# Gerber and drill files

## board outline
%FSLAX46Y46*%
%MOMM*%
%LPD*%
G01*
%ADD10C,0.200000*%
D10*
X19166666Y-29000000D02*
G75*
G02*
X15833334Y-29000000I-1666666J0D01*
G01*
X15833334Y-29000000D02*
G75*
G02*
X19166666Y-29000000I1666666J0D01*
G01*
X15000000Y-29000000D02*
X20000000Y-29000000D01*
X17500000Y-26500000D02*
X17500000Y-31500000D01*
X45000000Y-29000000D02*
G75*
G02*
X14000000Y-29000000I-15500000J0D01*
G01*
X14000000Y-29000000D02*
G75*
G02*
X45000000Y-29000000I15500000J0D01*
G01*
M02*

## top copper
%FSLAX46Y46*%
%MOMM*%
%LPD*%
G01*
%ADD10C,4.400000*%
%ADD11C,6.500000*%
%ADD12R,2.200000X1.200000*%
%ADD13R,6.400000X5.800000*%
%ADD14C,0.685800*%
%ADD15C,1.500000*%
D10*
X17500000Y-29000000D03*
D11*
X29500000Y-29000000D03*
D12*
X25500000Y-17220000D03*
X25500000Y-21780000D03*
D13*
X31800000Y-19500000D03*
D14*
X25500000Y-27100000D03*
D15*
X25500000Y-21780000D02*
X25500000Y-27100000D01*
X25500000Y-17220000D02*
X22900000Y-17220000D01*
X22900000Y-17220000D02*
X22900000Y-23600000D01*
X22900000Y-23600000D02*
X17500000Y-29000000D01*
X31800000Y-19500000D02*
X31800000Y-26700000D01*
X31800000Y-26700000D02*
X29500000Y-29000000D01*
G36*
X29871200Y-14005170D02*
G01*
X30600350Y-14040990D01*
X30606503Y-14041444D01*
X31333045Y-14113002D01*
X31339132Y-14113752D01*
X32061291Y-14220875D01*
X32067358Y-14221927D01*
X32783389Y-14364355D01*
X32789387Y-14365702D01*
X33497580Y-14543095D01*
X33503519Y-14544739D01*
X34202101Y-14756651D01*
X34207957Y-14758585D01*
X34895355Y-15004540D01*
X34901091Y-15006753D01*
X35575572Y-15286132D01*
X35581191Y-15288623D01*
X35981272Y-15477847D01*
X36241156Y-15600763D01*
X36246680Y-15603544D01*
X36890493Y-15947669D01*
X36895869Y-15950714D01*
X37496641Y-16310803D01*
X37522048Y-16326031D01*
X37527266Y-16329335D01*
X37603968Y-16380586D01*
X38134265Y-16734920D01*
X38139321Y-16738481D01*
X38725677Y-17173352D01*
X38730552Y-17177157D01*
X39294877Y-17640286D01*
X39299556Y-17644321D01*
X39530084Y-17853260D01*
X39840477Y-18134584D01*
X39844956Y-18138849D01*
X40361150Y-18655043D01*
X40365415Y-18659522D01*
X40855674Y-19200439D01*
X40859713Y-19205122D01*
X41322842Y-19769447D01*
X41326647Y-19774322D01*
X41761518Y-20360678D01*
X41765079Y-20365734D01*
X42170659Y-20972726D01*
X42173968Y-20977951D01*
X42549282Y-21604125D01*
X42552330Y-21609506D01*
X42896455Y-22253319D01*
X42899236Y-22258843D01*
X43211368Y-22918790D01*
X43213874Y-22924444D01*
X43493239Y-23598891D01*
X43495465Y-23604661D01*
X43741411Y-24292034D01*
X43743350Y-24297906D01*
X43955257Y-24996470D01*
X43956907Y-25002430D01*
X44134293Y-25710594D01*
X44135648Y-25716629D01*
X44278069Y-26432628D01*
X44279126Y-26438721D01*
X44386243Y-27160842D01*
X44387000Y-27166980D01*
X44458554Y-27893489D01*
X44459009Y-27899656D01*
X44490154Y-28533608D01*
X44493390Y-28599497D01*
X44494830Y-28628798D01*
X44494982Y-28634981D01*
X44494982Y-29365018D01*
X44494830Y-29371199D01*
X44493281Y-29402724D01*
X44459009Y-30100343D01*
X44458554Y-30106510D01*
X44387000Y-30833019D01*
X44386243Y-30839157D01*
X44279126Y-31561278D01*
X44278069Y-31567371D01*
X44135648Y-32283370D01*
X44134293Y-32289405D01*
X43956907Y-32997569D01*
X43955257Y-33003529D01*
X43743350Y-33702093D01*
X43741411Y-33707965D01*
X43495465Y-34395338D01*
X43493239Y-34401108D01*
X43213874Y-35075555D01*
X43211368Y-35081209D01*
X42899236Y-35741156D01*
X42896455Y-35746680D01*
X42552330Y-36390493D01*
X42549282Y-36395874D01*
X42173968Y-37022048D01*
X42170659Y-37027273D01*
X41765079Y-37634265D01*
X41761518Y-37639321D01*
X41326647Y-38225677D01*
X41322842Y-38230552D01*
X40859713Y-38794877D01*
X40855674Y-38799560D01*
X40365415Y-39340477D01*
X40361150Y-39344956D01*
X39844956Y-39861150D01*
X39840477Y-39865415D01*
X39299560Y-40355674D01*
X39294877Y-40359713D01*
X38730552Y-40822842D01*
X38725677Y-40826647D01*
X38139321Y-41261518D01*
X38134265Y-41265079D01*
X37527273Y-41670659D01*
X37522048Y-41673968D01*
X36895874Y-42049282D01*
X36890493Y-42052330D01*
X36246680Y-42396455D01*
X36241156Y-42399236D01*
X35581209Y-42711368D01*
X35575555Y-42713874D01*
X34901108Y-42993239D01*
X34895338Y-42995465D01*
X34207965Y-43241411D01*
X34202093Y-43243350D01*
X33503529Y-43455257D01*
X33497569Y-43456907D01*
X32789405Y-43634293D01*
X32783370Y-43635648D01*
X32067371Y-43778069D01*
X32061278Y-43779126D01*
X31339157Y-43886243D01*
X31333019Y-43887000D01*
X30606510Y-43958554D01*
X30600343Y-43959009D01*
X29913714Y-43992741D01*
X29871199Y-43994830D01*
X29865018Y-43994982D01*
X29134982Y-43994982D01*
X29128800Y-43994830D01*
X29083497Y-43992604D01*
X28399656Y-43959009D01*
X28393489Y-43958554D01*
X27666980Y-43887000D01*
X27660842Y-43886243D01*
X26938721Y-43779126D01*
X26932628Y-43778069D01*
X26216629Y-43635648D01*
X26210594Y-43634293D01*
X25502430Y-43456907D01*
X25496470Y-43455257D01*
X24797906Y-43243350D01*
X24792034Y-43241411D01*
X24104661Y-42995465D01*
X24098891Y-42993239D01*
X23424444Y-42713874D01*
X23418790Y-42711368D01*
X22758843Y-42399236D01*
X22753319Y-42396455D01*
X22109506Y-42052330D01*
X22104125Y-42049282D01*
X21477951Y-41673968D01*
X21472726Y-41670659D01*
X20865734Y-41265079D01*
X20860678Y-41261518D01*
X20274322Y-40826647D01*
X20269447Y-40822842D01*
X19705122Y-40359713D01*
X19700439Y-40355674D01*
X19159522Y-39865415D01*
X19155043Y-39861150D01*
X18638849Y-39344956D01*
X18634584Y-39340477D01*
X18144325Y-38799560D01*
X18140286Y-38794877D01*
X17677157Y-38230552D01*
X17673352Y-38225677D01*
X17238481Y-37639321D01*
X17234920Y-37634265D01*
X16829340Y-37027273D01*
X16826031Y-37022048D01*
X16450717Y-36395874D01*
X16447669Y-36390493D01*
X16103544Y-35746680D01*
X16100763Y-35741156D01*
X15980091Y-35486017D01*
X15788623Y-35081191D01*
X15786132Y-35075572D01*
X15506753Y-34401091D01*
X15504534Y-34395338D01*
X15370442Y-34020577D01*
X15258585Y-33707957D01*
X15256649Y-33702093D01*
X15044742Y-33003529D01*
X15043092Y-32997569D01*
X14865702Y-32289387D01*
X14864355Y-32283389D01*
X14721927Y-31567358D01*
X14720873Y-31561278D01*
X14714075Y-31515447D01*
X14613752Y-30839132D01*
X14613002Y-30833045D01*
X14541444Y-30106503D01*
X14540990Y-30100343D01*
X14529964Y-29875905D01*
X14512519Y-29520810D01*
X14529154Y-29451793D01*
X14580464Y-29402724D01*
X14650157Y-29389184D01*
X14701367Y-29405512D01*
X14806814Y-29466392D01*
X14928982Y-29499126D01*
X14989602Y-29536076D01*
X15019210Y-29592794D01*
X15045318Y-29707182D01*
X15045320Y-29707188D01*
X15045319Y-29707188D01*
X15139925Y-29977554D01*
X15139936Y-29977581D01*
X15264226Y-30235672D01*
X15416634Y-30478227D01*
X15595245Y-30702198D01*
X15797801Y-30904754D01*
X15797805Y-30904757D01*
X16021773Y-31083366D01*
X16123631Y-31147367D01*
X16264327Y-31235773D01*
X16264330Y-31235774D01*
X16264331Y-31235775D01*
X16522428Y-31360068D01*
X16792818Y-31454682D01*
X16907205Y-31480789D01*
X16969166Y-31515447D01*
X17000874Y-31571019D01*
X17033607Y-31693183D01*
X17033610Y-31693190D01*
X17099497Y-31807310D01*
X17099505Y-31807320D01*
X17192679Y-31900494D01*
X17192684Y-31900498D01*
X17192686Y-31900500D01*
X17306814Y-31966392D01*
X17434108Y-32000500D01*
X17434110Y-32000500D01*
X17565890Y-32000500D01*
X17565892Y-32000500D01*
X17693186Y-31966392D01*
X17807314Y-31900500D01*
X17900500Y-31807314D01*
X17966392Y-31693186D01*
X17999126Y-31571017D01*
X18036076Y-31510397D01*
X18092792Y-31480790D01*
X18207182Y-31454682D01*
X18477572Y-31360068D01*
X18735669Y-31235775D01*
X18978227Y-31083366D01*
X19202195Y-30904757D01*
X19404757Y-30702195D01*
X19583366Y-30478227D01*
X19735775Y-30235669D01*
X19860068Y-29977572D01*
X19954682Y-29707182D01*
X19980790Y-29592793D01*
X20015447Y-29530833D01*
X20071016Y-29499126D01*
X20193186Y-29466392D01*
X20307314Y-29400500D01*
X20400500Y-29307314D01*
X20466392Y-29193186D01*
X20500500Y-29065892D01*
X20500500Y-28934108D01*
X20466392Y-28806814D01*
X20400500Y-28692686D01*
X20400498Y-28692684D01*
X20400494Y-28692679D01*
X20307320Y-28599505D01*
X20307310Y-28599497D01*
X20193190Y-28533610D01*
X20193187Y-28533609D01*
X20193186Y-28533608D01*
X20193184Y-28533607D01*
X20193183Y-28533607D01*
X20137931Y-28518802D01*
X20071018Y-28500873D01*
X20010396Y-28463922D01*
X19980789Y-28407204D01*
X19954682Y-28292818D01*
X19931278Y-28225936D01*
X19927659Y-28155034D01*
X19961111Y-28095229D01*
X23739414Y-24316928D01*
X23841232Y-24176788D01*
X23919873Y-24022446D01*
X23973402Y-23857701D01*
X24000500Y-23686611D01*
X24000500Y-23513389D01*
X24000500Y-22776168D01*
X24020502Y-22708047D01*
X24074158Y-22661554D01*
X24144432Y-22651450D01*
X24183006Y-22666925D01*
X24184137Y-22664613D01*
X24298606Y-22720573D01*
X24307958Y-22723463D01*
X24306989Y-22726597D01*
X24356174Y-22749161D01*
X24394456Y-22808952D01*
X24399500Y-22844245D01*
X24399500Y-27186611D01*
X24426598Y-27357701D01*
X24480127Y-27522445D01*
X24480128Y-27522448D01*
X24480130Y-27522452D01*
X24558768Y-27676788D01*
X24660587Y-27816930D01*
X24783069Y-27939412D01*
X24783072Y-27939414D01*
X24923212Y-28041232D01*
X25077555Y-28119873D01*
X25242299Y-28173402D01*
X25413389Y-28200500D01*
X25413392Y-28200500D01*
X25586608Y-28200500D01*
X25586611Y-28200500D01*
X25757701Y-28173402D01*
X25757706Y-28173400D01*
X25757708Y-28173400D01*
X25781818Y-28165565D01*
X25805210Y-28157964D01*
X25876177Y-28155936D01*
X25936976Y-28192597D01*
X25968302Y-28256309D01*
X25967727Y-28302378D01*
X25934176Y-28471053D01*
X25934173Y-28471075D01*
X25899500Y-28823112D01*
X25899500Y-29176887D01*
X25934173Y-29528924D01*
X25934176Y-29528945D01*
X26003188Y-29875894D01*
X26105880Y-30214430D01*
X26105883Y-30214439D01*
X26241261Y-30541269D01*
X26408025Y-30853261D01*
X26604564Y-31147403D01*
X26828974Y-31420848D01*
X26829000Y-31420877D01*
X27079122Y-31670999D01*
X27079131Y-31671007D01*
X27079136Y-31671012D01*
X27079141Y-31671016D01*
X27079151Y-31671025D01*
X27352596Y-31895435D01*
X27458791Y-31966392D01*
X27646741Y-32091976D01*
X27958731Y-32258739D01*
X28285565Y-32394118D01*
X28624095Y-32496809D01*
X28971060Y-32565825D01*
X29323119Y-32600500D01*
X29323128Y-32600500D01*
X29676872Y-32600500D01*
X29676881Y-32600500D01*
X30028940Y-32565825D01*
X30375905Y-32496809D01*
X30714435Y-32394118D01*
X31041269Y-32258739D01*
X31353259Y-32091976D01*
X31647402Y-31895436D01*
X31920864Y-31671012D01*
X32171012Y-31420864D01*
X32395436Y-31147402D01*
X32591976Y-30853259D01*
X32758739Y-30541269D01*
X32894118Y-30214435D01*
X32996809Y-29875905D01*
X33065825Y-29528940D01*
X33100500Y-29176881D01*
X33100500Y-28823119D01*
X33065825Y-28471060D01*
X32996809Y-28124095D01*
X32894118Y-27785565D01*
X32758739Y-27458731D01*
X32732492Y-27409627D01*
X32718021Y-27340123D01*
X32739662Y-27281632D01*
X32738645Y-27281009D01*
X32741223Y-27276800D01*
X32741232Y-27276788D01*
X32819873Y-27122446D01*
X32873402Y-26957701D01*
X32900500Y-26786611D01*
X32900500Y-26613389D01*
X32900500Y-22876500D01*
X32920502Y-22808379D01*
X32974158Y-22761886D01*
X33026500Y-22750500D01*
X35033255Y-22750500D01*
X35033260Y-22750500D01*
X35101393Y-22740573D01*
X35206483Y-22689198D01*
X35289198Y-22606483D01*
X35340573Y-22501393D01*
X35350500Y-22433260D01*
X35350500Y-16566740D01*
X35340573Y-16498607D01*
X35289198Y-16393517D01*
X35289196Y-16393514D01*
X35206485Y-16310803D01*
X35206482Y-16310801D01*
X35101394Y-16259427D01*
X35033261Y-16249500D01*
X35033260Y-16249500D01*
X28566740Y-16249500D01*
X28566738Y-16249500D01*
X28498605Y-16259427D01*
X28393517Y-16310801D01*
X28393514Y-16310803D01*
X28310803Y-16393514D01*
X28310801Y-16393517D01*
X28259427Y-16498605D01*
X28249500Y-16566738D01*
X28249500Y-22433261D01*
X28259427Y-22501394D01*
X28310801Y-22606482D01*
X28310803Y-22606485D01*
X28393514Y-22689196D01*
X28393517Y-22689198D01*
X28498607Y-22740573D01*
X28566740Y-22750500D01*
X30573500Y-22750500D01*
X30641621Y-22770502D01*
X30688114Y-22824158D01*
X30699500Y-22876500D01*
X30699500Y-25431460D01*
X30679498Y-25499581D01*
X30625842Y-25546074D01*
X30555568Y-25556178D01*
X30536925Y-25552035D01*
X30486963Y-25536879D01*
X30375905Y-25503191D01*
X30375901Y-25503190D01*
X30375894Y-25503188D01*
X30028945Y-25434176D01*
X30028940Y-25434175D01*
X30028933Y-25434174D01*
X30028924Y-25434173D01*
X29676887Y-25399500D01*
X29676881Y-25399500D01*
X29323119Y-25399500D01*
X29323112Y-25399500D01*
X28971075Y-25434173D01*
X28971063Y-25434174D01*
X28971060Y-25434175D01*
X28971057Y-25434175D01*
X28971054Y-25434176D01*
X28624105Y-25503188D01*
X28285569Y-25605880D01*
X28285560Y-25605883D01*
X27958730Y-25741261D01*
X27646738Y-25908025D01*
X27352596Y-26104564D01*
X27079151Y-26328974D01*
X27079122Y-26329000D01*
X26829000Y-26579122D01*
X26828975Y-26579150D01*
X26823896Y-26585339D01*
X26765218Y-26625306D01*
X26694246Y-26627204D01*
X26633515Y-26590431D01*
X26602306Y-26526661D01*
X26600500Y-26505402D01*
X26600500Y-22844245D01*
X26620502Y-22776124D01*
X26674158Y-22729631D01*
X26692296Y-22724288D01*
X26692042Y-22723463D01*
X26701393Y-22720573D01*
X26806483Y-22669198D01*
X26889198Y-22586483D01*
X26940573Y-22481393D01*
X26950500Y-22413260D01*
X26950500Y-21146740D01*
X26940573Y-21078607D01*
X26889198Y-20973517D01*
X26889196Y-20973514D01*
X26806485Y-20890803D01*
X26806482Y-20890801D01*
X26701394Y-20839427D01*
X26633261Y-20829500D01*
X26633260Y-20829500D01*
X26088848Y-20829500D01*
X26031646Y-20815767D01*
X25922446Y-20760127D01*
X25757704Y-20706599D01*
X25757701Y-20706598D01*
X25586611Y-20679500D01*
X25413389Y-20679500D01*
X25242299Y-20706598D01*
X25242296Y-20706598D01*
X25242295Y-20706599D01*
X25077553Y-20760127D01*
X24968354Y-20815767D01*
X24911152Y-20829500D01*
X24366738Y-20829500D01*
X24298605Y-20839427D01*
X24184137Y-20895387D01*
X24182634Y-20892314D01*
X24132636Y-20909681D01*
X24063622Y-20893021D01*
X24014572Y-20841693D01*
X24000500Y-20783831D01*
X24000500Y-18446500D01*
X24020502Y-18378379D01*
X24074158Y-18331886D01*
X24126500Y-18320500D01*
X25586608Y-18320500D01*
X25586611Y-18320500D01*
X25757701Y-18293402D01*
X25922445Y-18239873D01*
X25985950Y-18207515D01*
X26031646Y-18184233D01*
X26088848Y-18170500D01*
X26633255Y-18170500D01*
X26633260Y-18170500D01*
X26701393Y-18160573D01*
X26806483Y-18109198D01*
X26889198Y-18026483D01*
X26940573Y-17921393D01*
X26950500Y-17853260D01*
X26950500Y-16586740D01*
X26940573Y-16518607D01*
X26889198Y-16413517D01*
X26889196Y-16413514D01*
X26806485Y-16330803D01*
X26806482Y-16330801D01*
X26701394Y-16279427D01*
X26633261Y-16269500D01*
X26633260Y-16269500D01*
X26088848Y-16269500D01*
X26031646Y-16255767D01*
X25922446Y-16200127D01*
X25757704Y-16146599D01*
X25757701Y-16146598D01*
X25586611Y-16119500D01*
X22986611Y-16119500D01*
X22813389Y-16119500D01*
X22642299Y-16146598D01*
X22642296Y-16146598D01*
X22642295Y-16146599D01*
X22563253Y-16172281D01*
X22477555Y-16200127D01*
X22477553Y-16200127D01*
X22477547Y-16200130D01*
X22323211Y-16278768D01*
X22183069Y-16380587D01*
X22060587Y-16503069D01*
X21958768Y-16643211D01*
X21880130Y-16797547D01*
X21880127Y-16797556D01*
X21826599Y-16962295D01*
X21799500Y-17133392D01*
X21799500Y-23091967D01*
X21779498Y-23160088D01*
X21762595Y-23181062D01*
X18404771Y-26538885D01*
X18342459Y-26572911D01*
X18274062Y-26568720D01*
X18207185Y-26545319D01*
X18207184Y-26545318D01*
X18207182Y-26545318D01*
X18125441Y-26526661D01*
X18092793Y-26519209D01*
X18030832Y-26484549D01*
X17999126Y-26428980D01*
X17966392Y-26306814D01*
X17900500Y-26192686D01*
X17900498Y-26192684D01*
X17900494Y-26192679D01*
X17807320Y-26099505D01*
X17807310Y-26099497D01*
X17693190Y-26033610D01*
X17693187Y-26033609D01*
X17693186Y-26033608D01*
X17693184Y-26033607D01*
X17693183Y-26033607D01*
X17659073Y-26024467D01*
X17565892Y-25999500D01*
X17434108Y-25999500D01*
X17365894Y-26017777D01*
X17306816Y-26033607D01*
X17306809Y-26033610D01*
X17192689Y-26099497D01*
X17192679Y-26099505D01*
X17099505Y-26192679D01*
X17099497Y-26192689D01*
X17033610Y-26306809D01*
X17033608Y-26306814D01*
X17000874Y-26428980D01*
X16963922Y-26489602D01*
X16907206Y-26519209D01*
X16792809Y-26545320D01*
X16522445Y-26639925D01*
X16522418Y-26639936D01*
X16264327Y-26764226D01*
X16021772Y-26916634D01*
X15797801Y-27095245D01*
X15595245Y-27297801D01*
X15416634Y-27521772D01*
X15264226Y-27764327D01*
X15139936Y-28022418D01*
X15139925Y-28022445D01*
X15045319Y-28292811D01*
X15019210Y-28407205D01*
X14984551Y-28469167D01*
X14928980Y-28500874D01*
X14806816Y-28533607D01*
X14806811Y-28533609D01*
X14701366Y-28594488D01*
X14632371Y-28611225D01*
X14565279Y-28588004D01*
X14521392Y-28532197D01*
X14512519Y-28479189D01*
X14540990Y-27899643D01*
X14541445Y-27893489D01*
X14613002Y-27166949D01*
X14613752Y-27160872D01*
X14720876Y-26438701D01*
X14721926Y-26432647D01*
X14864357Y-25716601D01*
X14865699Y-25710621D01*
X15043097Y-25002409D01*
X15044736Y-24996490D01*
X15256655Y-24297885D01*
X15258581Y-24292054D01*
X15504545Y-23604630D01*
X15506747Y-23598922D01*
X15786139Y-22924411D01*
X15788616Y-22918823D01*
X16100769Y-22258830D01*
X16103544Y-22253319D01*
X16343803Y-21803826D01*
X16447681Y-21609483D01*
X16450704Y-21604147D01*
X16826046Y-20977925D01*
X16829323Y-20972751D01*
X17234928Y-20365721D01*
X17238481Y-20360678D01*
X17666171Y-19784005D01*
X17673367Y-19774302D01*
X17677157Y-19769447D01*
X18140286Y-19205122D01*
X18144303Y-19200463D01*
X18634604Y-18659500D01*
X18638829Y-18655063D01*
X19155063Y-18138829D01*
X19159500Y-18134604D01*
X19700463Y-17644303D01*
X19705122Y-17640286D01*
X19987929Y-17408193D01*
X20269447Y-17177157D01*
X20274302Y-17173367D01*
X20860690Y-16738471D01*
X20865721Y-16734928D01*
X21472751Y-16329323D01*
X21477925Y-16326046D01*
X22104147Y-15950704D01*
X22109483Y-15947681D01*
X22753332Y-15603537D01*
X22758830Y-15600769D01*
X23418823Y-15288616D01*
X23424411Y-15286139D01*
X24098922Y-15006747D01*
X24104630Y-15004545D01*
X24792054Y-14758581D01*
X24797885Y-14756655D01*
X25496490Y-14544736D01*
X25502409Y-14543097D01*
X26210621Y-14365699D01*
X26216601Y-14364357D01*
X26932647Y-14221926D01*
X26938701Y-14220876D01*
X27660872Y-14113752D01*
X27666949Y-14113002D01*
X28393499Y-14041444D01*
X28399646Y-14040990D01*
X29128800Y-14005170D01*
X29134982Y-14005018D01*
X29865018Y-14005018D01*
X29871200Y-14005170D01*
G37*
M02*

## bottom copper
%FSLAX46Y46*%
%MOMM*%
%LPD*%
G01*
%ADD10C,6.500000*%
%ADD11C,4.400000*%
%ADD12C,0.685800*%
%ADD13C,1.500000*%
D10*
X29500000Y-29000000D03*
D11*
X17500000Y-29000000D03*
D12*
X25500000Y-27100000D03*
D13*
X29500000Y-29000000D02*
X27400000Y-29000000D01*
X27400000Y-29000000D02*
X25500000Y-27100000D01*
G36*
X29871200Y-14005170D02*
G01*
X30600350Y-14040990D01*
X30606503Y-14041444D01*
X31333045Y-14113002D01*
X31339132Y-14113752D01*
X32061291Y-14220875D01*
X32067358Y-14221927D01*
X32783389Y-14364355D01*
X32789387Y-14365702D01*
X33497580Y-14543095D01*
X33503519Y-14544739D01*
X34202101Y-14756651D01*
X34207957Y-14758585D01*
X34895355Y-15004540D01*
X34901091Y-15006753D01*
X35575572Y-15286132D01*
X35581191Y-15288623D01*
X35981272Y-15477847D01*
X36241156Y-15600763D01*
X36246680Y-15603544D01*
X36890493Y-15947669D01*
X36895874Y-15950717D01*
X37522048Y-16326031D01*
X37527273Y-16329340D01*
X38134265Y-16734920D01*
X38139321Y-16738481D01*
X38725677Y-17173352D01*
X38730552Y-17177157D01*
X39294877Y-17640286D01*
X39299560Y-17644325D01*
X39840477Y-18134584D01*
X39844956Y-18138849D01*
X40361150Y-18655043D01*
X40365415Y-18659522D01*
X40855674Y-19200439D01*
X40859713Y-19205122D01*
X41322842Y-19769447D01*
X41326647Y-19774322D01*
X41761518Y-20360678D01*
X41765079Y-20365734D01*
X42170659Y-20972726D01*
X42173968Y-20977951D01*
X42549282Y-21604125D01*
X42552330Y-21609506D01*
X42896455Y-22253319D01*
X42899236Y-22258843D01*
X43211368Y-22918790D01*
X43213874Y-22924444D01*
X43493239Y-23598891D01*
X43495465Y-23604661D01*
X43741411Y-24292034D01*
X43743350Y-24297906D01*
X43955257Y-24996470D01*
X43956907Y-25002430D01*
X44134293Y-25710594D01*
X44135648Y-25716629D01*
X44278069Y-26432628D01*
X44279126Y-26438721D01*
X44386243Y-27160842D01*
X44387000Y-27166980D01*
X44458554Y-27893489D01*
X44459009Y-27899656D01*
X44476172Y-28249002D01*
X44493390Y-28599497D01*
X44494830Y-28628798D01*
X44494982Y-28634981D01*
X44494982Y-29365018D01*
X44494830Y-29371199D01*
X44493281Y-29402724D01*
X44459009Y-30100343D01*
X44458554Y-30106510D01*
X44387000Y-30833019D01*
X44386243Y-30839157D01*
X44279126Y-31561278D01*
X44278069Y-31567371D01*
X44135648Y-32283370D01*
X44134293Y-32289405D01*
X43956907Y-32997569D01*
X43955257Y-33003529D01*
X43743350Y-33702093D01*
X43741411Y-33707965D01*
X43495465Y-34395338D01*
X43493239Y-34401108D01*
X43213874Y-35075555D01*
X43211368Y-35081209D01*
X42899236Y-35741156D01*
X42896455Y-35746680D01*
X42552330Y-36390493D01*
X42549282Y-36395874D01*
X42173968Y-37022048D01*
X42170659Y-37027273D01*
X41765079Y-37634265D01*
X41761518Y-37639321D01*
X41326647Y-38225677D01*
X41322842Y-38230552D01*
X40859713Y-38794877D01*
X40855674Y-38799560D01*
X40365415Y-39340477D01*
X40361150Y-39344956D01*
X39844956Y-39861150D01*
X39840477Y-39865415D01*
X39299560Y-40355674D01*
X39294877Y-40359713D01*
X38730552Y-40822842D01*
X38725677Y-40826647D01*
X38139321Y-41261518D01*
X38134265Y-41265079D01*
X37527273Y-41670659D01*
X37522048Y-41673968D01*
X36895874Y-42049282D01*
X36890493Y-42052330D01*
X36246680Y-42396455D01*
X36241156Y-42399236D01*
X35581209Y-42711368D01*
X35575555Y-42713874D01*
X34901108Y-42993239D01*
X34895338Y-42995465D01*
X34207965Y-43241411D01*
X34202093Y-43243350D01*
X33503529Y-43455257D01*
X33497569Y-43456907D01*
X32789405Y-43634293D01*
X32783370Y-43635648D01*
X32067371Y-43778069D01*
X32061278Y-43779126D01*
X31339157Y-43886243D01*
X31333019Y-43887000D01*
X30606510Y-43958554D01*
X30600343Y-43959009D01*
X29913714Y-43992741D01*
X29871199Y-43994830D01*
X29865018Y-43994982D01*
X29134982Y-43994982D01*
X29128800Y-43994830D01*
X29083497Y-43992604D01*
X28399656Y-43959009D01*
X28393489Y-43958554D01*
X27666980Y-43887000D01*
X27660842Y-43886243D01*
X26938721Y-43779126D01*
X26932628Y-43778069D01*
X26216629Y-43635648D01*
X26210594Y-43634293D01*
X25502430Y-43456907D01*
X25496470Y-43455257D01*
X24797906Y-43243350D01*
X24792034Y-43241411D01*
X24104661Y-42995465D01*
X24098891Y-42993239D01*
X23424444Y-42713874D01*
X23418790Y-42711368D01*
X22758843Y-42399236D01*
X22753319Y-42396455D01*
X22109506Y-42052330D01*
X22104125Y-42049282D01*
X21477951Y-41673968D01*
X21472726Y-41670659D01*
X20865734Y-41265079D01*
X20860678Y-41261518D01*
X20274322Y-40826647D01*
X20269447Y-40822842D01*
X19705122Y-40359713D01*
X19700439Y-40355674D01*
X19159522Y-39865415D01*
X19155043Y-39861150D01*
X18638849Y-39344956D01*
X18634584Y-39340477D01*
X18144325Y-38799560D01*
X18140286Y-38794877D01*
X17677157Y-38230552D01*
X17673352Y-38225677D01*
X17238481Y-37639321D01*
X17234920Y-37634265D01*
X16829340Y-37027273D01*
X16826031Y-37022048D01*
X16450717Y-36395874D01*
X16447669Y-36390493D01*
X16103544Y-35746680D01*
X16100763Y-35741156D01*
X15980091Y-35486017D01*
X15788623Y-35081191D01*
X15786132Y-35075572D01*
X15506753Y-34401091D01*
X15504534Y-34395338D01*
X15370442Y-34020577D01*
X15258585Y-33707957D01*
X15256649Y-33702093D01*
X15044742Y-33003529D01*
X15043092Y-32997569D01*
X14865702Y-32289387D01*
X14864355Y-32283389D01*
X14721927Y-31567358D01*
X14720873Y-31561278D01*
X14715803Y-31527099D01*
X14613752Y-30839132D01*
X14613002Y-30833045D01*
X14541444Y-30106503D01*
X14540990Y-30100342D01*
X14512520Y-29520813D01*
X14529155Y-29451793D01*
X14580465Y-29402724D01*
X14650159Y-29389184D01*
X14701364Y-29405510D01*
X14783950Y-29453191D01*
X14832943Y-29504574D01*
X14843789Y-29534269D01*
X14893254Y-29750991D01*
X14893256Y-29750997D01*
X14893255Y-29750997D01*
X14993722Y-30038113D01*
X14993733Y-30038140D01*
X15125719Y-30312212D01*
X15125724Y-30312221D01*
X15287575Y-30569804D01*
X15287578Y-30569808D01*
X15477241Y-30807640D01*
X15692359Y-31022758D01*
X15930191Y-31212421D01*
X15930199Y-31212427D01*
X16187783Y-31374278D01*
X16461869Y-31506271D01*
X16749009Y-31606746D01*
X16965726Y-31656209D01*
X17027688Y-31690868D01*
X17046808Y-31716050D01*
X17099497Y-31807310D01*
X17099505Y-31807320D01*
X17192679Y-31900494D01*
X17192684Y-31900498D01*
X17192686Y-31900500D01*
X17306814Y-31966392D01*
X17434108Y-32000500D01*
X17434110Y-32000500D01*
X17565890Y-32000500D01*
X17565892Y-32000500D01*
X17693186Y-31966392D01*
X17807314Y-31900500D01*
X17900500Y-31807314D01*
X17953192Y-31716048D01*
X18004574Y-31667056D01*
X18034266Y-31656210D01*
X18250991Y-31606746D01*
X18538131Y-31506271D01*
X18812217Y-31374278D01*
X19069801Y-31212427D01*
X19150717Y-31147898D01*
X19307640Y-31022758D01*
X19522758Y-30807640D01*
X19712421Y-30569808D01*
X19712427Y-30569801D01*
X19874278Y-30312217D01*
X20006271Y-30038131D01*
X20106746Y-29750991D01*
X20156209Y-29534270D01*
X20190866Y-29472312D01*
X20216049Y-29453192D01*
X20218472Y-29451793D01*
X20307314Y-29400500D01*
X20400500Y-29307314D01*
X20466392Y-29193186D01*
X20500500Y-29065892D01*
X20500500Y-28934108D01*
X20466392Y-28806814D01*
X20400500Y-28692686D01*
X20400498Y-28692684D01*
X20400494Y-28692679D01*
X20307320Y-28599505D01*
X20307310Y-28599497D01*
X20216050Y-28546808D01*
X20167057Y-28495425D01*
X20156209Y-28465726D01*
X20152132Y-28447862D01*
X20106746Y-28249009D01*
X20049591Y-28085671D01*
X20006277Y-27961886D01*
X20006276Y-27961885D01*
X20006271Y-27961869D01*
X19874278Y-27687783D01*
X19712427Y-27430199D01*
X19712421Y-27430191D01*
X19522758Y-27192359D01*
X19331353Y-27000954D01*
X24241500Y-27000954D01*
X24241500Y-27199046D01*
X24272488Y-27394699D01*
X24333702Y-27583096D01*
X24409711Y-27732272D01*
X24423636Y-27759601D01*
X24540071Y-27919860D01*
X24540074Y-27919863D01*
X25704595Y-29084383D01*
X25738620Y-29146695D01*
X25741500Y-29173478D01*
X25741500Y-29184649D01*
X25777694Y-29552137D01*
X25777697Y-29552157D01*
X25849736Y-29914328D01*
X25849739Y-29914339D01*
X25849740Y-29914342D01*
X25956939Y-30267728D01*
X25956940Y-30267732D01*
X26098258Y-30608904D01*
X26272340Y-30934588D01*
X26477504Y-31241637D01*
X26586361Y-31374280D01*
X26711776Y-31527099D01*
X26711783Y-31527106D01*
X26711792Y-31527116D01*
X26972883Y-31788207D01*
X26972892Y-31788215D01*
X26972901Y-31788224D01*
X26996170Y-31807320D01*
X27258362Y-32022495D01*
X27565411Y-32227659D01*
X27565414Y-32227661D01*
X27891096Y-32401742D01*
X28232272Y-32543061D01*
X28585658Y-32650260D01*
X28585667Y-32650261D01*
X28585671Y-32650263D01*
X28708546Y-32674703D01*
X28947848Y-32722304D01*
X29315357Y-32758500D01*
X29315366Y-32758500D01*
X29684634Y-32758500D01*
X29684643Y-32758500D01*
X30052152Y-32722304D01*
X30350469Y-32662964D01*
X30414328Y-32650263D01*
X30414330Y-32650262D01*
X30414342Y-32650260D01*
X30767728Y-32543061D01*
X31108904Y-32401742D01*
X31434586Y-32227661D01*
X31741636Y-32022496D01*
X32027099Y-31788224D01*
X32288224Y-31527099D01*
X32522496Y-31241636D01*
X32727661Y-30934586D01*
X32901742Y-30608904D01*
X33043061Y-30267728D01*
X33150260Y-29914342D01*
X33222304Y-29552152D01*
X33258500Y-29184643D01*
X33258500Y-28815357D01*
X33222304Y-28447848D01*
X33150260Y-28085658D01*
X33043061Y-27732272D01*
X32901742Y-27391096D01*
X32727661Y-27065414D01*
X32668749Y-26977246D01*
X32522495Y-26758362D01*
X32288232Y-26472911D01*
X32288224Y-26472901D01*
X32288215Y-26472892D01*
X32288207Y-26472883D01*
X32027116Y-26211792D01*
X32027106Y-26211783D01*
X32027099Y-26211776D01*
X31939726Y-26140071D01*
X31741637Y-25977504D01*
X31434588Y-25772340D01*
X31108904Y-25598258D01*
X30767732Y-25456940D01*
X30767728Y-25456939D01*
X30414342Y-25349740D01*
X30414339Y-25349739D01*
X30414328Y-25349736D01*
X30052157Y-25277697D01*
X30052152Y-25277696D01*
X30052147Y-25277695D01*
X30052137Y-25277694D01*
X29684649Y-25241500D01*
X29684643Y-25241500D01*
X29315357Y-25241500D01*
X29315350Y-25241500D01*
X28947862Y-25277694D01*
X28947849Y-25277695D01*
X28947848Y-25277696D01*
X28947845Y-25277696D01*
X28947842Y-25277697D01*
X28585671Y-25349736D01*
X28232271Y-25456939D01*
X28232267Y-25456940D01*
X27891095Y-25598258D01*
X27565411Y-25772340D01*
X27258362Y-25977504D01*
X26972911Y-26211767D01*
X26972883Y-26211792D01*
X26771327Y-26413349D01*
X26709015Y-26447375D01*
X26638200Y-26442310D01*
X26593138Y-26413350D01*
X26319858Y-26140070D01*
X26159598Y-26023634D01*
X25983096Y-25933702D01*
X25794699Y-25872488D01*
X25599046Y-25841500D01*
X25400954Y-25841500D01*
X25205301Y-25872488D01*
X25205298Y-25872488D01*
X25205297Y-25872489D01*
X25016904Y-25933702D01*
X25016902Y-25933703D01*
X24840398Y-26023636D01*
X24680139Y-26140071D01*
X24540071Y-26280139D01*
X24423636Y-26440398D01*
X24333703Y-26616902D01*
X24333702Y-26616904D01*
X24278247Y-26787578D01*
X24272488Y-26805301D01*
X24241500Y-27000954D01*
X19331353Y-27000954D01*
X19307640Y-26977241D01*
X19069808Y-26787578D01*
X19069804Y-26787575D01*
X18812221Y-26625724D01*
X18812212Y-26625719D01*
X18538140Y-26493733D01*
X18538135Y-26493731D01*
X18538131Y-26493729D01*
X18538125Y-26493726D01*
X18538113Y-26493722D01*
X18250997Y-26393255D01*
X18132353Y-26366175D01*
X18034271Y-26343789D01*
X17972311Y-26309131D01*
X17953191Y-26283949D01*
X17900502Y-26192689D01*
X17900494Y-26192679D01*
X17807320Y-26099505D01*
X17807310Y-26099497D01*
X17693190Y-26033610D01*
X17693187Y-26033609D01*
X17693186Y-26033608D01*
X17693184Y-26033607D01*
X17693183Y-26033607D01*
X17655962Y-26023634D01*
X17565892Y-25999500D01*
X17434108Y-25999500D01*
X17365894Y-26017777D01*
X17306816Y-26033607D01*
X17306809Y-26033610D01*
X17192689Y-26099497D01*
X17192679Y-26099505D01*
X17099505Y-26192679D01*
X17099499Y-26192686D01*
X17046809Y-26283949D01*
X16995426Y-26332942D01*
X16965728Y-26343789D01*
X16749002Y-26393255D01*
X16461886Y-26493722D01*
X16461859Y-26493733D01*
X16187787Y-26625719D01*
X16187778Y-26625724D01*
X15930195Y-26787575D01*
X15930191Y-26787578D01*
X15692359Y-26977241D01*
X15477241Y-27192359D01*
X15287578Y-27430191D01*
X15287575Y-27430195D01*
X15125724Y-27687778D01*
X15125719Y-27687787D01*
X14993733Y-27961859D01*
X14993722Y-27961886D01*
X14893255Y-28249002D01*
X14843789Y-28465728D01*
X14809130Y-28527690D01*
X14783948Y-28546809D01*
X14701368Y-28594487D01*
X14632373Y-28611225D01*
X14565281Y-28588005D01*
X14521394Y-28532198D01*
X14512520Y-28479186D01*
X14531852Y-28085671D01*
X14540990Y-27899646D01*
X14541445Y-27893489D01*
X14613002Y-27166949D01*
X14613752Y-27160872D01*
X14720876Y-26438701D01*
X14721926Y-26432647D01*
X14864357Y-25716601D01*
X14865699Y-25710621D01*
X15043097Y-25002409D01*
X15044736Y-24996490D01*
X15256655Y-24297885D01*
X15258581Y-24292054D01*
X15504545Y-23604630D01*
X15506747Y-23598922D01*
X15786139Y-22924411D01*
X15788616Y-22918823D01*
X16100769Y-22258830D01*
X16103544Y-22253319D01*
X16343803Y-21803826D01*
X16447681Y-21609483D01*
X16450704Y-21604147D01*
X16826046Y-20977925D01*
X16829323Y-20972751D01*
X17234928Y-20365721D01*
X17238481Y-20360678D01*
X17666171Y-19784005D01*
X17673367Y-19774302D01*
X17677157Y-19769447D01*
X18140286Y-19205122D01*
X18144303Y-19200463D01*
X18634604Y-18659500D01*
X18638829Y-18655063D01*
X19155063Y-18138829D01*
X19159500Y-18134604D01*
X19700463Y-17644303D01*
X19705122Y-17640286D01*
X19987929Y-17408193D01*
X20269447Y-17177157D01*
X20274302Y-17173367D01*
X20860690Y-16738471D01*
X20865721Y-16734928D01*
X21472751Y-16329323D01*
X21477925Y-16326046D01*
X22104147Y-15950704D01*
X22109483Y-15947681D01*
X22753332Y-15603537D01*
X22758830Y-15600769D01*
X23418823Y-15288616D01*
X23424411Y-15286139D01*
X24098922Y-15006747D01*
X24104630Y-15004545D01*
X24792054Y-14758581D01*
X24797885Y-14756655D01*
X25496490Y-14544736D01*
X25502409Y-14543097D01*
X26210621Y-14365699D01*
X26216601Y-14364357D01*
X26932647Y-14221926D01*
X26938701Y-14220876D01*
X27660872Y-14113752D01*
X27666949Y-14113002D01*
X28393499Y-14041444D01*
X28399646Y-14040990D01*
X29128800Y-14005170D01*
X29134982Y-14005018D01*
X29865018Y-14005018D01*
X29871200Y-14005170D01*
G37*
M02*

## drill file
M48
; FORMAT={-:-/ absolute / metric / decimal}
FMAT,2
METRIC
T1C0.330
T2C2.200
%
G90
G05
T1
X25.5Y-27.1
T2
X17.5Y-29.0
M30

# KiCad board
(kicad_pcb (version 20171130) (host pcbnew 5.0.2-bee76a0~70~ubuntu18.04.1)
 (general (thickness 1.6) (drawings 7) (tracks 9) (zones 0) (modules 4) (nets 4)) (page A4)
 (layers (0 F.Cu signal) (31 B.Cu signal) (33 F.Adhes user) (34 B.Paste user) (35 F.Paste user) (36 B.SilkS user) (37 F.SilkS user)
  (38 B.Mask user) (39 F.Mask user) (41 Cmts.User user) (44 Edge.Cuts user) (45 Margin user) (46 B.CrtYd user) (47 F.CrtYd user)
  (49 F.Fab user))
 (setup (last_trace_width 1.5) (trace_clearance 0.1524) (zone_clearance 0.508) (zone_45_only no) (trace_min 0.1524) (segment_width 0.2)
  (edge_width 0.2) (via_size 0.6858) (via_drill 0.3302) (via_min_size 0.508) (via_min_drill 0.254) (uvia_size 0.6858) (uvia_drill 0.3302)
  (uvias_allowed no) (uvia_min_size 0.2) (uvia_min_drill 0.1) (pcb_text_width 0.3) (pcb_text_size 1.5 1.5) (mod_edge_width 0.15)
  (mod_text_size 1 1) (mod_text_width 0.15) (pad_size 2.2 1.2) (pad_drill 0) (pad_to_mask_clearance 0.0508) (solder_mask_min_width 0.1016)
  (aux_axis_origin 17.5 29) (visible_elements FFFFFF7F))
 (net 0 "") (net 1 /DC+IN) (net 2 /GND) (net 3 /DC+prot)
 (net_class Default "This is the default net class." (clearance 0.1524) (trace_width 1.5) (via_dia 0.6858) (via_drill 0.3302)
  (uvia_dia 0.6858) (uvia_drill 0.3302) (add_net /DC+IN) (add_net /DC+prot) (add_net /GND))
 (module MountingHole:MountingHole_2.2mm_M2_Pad (layer F.Cu) (at 29.5 29)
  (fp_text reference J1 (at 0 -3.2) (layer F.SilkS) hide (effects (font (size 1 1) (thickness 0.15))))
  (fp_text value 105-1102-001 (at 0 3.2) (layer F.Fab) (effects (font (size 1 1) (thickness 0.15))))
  (pad 1 smd circle (at 0 0) (size 6.5 6.5) (layers B.Cu F.Paste F.Mask) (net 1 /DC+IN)))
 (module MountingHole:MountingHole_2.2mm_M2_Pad (layer F.Cu) (at 17.5 29)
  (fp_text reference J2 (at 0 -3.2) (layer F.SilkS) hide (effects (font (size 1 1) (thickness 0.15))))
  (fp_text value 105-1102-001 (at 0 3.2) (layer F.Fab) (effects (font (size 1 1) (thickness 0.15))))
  (pad 1 thru_hole circle (at 0 0) (size 4.4 4.4) (drill 2.2) (layers *.Cu *.Mask) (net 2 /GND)))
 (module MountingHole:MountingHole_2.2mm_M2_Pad (layer F.Cu) (at 29.5 29)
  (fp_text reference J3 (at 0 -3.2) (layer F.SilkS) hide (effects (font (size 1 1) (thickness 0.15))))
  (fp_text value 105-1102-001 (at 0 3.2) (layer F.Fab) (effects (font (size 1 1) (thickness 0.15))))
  (pad 1 smd circle (at 0 0) (size 6.5 6.5) (layers F.Cu F.Paste F.Mask) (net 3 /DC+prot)))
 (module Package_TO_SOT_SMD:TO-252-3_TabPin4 (layer F.Cu) (at 29.7 19.5)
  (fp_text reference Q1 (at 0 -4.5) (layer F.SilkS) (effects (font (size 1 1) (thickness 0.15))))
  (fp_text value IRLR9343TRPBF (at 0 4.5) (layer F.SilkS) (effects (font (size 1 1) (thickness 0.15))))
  (pad 1 smd rect (at -4.2 -2.28) (size 2.2 1.2) (layers F.Cu F.Paste F.Mask) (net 2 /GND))
  (pad 2 smd rect (at -4.2 0) (size 2.2 1.2) (layers F.Paste F.Mask))
  (pad 3 smd rect (at -4.2 2.28) (size 2.2 1.2) (layers F.Cu F.Paste F.Mask))
  (pad 4 smd rect (at 2.1 0) (size 6.4 5.8) (layers F.Cu F.Mask) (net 3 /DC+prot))
  (pad "" smd rect (at 3.775 1.525) (size 3.05 2.75) (layers F.Paste))
  (pad "" smd rect (at 0.425 -1.525) (size 3.05 2.75) (layers F.Paste))
  (pad "" smd rect (at 3.775 -1.525) (size 3.05 2.75) (layers F.Paste))
  (pad "" smd rect (at 0.425 1.525) (size 3.05 2.75) (layers F.Paste)))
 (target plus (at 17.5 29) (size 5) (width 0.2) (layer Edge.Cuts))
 (gr_circle (center 29.5 29) (end 45 29) (layer Edge.Cuts) (width 0.2))
 (segment (start 25.5 21.78) (end 25.5 27.1) (width 1.5) (layer F.Cu) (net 1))
 (segment (start 29.5 29) (end 27.4 29) (width 1.5) (layer B.Cu) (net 1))
 (segment (start 27.4 29) (end 25.5 27.1) (width 1.5) (layer B.Cu) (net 1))
 (via (at 25.5 27.1) (size 0.6858) (layers F.Cu B.Cu) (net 1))
 (segment (start 25.5 17.22) (end 22.9 17.22) (width 1.5) (layer F.Cu) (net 2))
 (segment (start 22.9 17.22) (end 22.9 23.6) (width 1.5) (layer F.Cu) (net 2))
 (segment (start 22.9 23.6) (end 17.5 29) (width 1.5) (layer F.Cu) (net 2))
 (segment (start 31.8 19.5) (end 31.8 26.7) (width 1.5) (layer F.Cu) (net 3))
 (segment (start 31.8 26.7) (end 29.5 29) (width 1.5) (layer F.Cu) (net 3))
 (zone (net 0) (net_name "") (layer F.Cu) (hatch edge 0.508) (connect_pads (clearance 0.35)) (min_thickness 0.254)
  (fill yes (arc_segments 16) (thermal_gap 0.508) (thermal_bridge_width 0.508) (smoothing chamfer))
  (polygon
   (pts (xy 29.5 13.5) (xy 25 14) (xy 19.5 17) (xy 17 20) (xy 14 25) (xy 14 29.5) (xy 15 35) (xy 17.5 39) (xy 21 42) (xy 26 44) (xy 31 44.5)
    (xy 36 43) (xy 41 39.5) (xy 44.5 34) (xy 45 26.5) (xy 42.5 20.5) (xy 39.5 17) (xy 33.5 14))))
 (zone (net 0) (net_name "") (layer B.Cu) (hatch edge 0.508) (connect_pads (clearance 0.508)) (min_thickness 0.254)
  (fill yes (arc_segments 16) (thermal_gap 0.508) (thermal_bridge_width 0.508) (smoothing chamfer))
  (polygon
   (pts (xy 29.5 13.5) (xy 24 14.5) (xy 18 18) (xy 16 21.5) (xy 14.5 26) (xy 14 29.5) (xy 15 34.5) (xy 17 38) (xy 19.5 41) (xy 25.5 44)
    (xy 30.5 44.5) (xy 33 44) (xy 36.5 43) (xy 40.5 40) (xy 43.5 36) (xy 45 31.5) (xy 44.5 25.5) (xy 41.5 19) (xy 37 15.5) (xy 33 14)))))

